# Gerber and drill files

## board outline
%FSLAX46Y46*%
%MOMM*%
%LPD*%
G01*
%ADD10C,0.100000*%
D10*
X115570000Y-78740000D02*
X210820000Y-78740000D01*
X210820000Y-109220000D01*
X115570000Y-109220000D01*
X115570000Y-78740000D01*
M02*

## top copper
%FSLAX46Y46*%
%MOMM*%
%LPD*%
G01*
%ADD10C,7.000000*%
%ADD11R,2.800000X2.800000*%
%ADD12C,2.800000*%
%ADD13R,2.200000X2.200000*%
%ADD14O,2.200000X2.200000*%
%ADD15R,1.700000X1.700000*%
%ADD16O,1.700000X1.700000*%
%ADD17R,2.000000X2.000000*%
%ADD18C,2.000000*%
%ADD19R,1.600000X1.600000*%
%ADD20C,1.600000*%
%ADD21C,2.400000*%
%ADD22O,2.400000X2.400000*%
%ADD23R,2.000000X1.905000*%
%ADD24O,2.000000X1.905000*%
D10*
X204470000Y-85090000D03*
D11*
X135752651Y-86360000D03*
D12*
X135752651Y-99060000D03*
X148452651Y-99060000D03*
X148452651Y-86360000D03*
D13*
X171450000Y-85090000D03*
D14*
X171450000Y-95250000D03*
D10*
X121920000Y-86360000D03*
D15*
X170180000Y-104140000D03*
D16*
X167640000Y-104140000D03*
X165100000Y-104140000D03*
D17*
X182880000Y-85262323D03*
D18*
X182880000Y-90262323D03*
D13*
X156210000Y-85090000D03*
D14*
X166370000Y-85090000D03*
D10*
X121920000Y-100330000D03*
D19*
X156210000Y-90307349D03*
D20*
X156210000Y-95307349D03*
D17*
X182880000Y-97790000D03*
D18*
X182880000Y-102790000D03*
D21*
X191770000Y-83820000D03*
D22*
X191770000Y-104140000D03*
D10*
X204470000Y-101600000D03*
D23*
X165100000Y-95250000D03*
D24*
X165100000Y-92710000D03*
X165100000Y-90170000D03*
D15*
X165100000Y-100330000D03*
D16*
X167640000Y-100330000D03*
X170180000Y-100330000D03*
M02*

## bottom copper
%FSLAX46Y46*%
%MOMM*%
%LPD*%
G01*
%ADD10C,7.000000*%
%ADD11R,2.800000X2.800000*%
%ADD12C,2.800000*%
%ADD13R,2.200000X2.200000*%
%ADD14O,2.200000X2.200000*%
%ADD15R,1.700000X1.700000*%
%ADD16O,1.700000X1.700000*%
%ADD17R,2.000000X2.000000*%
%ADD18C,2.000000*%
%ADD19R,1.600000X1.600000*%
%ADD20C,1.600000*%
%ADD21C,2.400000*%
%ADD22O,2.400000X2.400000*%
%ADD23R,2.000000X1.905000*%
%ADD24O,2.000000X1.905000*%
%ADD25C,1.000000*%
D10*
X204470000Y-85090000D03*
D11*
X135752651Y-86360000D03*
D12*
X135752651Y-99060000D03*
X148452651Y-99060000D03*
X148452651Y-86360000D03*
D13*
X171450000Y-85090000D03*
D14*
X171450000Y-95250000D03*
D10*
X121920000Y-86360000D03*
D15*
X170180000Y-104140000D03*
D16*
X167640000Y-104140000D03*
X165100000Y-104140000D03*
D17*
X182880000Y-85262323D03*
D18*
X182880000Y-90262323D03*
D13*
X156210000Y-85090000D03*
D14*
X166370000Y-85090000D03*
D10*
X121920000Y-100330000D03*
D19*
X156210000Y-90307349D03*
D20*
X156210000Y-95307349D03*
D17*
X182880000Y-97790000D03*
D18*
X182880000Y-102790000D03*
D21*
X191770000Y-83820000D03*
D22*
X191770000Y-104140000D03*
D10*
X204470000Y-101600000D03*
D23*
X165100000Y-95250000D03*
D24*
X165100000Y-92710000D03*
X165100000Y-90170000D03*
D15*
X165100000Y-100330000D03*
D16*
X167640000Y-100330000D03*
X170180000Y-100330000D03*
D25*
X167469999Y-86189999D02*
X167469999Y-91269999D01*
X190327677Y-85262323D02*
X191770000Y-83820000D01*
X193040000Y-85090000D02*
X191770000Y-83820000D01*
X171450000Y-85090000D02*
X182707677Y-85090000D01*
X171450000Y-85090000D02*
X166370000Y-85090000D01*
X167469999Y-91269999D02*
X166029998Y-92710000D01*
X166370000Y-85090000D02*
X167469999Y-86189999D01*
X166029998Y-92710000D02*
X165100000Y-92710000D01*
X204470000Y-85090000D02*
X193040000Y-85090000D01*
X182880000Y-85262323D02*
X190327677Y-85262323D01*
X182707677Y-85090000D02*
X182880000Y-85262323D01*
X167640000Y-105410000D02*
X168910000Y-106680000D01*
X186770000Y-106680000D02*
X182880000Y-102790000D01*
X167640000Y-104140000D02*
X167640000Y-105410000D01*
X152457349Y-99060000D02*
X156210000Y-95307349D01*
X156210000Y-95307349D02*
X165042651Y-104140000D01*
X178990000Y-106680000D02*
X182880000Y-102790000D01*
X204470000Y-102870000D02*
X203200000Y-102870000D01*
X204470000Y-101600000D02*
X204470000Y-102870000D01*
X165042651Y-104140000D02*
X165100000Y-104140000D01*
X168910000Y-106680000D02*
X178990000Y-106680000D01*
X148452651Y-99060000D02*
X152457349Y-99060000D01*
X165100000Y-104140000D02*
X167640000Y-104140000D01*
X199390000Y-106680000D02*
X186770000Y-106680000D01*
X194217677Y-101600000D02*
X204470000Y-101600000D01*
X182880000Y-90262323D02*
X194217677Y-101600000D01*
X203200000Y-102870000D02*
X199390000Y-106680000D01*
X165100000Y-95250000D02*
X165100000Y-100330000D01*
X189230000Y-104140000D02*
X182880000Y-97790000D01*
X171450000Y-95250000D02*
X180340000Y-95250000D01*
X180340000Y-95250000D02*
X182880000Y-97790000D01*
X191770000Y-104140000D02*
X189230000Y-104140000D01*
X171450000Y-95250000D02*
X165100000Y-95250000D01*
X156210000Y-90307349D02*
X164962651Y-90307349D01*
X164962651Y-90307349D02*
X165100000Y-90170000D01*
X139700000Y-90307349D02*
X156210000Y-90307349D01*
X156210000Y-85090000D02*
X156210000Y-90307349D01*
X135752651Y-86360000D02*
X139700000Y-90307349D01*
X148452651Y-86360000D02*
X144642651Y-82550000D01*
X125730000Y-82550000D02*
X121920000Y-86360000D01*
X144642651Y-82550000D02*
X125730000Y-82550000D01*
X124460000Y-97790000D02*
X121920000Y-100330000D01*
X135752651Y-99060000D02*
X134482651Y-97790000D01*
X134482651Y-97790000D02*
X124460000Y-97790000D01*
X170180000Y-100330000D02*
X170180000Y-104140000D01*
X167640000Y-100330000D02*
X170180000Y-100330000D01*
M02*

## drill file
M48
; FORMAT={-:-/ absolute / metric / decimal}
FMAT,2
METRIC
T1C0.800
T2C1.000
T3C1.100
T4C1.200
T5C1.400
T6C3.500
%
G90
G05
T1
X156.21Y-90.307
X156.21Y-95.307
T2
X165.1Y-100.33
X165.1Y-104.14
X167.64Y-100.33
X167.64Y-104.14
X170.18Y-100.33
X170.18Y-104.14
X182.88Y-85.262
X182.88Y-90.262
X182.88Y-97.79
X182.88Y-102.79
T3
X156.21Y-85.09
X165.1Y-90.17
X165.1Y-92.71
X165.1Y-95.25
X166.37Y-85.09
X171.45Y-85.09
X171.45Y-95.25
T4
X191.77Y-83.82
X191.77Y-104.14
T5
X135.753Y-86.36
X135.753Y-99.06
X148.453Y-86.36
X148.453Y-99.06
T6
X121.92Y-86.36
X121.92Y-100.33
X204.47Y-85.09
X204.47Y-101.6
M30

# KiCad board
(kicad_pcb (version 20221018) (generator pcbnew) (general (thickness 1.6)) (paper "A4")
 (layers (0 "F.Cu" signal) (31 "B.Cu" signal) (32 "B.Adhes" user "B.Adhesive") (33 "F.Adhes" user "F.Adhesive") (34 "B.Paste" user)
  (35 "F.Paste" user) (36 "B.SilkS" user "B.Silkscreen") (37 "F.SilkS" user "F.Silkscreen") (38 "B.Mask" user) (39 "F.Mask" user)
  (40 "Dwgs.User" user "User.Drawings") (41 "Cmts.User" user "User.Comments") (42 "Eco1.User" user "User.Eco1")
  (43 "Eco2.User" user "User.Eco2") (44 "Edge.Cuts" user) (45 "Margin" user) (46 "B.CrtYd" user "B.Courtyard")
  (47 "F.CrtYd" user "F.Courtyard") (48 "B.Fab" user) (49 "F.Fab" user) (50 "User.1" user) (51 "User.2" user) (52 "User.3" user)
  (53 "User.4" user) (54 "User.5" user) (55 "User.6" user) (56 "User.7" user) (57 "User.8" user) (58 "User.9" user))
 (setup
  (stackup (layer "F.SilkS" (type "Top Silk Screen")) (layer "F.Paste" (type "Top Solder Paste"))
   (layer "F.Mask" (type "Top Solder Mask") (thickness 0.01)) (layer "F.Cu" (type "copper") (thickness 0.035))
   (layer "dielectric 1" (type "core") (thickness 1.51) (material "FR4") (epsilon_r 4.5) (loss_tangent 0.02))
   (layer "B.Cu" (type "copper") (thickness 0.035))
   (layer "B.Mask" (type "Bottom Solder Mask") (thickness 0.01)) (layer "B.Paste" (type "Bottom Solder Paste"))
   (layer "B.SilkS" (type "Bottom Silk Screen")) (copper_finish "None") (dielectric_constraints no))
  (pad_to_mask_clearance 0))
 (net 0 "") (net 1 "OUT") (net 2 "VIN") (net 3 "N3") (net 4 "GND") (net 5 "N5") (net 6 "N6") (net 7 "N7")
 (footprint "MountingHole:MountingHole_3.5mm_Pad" (layer "F.Cu") (at 204.47 85.09)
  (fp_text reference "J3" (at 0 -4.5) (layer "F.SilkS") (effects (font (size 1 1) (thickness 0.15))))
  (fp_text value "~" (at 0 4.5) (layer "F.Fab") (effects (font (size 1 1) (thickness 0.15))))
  (pad "1" thru_hole circle (at 0 0) (size 7 7) (drill 3.5) (layers "*.Cu" "*.Mask") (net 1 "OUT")))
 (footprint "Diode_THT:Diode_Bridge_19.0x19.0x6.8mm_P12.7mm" (layer "F.Cu") (at 135.752651 86.36)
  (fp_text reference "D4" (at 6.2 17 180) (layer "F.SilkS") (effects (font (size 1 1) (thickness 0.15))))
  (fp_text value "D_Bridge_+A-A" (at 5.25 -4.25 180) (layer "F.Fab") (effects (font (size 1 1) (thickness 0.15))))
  (pad "1" thru_hole rect (at 0 0 180) (size 2.8 2.8) (drill 1.4) (layers "*.Cu" "*.Mask") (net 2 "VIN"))
  (pad "2" thru_hole circle (at 0 12.7 180) (size 2.8 2.8) (drill 1.4) (layers "*.Cu" "*.Mask") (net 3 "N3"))
  (pad "3" thru_hole circle (at 12.7 12.7 180) (size 2.8 2.8) (drill 1.4) (layers "*.Cu" "*.Mask") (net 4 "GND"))
  (pad "4" thru_hole circle (at 12.7 0 180) (size 2.8 2.8) (drill 1.4) (layers "*.Cu" "*.Mask") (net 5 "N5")))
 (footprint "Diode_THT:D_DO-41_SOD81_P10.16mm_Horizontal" (layer "F.Cu") (at 171.45 85.09 -90)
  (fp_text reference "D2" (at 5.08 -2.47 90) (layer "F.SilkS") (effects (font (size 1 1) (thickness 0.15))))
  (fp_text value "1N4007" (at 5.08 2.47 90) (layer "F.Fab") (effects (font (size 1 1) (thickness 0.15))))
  (pad "1" thru_hole rect (at 0 0 270) (size 2.2 2.2) (drill 1.1) (layers "*.Cu" "*.Mask") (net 1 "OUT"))
  (pad "2" thru_hole oval (at 10.16 0 270) (size 2.2 2.2) (drill 1.1) (layers "*.Cu" "*.Mask") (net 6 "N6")))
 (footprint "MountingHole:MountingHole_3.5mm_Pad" (layer "F.Cu") (at 121.92 86.36)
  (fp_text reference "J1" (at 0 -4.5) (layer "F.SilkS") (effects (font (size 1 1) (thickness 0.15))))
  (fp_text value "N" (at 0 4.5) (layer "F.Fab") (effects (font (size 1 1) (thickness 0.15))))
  (pad "1" thru_hole circle (at 0 0) (size 7 7) (drill 3.5) (layers "*.Cu" "*.Mask") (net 5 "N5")))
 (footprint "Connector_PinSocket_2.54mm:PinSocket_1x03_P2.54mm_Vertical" (layer "F.Cu") (at 170.18 104.14 -90)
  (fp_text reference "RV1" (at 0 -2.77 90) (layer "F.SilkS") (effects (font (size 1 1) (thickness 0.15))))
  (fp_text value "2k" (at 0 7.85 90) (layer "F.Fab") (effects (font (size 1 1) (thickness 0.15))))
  (pad "1" thru_hole rect (at 0 0 270) (size 1.7 1.7) (drill 1) (layers "*.Cu" "*.Mask") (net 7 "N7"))
  (pad "2" thru_hole oval (at 0 2.54 270) (size 1.7 1.7) (drill 1) (layers "*.Cu" "*.Mask") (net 4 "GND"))
  (pad "3" thru_hole oval (at 0 5.08 270) (size 1.7 1.7) (drill 1) (layers "*.Cu" "*.Mask") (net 4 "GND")))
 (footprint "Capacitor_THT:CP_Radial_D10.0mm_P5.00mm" (layer "F.Cu") (at 182.88 85.262323 -90)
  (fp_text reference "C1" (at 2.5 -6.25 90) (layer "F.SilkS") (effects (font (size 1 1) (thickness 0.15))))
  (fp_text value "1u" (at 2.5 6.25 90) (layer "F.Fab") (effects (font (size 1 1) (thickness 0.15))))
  (pad "1" thru_hole rect (at 0 0 270) (size 2 2) (drill 1) (layers "*.Cu" "*.Mask") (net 1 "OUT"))
  (pad "2" thru_hole circle (at 5 0 270) (size 2 2) (drill 1) (layers "*.Cu" "*.Mask") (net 4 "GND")))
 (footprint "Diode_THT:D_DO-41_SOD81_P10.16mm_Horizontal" (layer "F.Cu") (at 156.21 85.09)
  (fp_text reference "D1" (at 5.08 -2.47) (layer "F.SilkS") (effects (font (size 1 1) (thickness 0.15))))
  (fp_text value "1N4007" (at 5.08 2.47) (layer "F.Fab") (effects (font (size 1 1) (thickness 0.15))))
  (pad "1" thru_hole rect (at 0 0) (size 2.2 2.2) (drill 1.1) (layers "*.Cu" "*.Mask") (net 2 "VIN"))
  (pad "2" thru_hole oval (at 10.16 0) (size 2.2 2.2) (drill 1.1) (layers "*.Cu" "*.Mask") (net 1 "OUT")))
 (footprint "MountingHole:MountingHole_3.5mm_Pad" (layer "F.Cu") (at 121.92 100.33)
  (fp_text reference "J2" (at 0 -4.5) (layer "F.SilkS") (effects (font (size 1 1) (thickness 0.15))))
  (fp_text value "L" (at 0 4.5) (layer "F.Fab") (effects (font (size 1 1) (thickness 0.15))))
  (pad "1" thru_hole circle (at 0 0) (size 7 7) (drill 3.5) (layers "*.Cu" "*.Mask") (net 3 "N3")))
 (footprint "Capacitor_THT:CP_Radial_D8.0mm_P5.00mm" (layer "F.Cu") (at 156.21 90.307349 -90)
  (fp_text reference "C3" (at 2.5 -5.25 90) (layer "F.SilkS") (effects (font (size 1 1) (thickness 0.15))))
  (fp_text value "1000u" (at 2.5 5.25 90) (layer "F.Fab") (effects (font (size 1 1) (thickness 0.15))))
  (pad "1" thru_hole rect (at 0 0 270) (size 1.6 1.6) (drill 0.8) (layers "*.Cu" "*.Mask") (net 2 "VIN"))
  (pad "2" thru_hole circle (at 5 0 270) (size 1.6 1.6) (drill 0.8) (layers "*.Cu" "*.Mask") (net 4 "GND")))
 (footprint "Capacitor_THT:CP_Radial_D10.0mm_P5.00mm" (layer "F.Cu") (at 182.88 97.79 -90)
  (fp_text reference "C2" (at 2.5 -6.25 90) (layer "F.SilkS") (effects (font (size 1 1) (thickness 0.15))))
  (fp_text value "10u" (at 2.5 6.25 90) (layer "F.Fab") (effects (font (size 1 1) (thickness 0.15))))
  (pad "1" thru_hole rect (at 0 0 270) (size 2 2) (drill 1) (layers "*.Cu" "*.Mask") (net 6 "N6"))
  (pad "2" thru_hole circle (at 5 0 270) (size 2 2) (drill 1) (layers "*.Cu" "*.Mask") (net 4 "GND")))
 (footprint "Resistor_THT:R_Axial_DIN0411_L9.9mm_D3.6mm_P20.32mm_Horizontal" (layer "F.Cu") (at 191.77 83.82 -90)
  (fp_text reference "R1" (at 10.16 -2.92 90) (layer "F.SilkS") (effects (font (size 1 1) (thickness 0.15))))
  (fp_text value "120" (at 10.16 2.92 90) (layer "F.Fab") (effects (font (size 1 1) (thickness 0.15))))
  (pad "1" thru_hole circle (at 0 0 270) (size 2.4 2.4) (drill 1.2) (layers "*.Cu" "*.Mask") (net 1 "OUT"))
  (pad "2" thru_hole oval (at 20.32 0 270) (size 2.4 2.4) (drill 1.2) (layers "*.Cu" "*.Mask") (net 6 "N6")))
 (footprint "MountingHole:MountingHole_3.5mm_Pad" (layer "F.Cu") (at 204.47 101.6)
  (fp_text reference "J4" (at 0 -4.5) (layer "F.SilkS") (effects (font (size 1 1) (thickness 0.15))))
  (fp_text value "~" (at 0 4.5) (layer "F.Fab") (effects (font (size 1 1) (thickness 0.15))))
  (pad "1" thru_hole circle (at 0 0) (size 7 7) (drill 3.5) (layers "*.Cu" "*.Mask") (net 4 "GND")))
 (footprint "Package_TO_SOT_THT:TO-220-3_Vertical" (layer "F.Cu") (at 165.1 95.25 90)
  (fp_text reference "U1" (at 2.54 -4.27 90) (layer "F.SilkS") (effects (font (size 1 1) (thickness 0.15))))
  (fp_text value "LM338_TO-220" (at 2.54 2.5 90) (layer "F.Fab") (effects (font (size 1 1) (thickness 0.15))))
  (pad "1" thru_hole rect (at 0 0 90) (size 1.905 2) (drill 1.1) (layers "*.Cu" "*.Mask") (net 6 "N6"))
  (pad "2" thru_hole oval (at 2.54 0 90) (size 1.905 2) (drill 1.1) (layers "*.Cu" "*.Mask") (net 1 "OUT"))
  (pad "3" thru_hole oval (at 5.08 0 90) (size 1.905 2) (drill 1.1) (layers "*.Cu" "*.Mask") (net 2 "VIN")))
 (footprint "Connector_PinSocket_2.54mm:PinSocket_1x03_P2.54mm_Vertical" (layer "F.Cu") (at 165.1 100.33 90)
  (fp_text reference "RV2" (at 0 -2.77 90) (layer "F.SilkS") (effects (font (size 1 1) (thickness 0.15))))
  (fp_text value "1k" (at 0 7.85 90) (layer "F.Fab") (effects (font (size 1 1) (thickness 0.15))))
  (pad "1" thru_hole rect (at 0 0 90) (size 1.7 1.7) (drill 1) (layers "*.Cu" "*.Mask") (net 6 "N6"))
  (pad "2" thru_hole oval (at 0 2.54 90) (size 1.7 1.7) (drill 1) (layers "*.Cu" "*.Mask") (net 7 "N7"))
  (pad "3" thru_hole oval (at 0 5.08 90) (size 1.7 1.7) (drill 1) (layers "*.Cu" "*.Mask") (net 7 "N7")))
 (gr_rect (start 115.57 78.74) (end 210.82 109.22) (stroke (width 0.1) (type default)) (fill none) (layer "Edge.Cuts"))
 (segment (start 167.469999 86.189999) (end 167.469999 91.269999) (width 1) (layer "B.Cu") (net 1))
 (segment (start 190.327677 85.262323) (end 191.77 83.82) (width 1) (layer "B.Cu") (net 1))
 (segment (start 193.04 85.09) (end 191.77 83.82) (width 1) (layer "B.Cu") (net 1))
 (segment (start 171.45 85.09) (end 182.707677 85.09) (width 1) (layer "B.Cu") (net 1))
 (segment (start 171.45 85.09) (end 166.37 85.09) (width 1) (layer "B.Cu") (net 1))
 (segment (start 167.469999 91.269999) (end 166.029998 92.71) (width 1) (layer "B.Cu") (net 1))
 (segment (start 166.37 85.09) (end 167.469999 86.189999) (width 1) (layer "B.Cu") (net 1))
 (segment (start 166.029998 92.71) (end 165.1 92.71) (width 1) (layer "B.Cu") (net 1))
 (segment (start 204.47 85.09) (end 193.04 85.09) (width 1) (layer "B.Cu") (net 1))
 (segment (start 182.88 85.262323) (end 190.327677 85.262323) (width 1) (layer "B.Cu") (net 1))
 (segment (start 182.707677 85.09) (end 182.88 85.262323) (width 1) (layer "B.Cu") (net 1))
 (segment (start 167.64 105.41) (end 168.91 106.68) (width 1) (layer "B.Cu") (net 4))
 (segment (start 186.77 106.68) (end 182.88 102.79) (width 1) (layer "B.Cu") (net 4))
 (segment (start 167.64 104.14) (end 167.64 105.41) (width 1) (layer "B.Cu") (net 4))
 (segment (start 152.457349 99.06) (end 156.21 95.307349) (width 1) (layer "B.Cu") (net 4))
 (segment (start 156.21 95.307349) (end 165.042651 104.14) (width 1) (layer "B.Cu") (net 4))
 (segment (start 178.99 106.68) (end 182.88 102.79) (width 1) (layer "B.Cu") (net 4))
 (segment (start 204.47 102.87) (end 203.2 102.87) (width 1) (layer "B.Cu") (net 4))
 (segment (start 204.47 101.6) (end 204.47 102.87) (width 1) (layer "B.Cu") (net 4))
 (segment (start 165.042651 104.14) (end 165.1 104.14) (width 1) (layer "B.Cu") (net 4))
 (segment (start 168.91 106.68) (end 178.99 106.68) (width 1) (layer "B.Cu") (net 4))
 (segment (start 148.452651 99.06) (end 152.457349 99.06) (width 1) (layer "B.Cu") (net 4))
 (segment (start 165.1 104.14) (end 167.64 104.14) (width 1) (layer "B.Cu") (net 4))
 (segment (start 199.39 106.68) (end 186.77 106.68) (width 1) (layer "B.Cu") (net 4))
 (segment (start 194.217677 101.6) (end 204.47 101.6) (width 1) (layer "B.Cu") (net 4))
 (segment (start 182.88 90.262323) (end 194.217677 101.6) (width 1) (layer "B.Cu") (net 4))
 (segment (start 203.2 102.87) (end 199.39 106.68) (width 1) (layer "B.Cu") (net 4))
 (segment (start 165.1 95.25) (end 165.1 100.33) (width 1) (layer "B.Cu") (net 6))
 (segment (start 189.23 104.14) (end 182.88 97.79) (width 1) (layer "B.Cu") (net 6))
 (segment (start 171.45 95.25) (end 180.34 95.25) (width 1) (layer "B.Cu") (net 6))
 (segment (start 180.34 95.25) (end 182.88 97.79) (width 1) (layer "B.Cu") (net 6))
 (segment (start 191.77 104.14) (end 189.23 104.14) (width 1) (layer "B.Cu") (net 6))
 (segment (start 171.45 95.25) (end 165.1 95.25) (width 1) (layer "B.Cu") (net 6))
 (segment (start 156.21 90.307349) (end 164.962651 90.307349) (width 1) (layer "B.Cu") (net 2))
 (segment (start 164.962651 90.307349) (end 165.1 90.17) (width 1) (layer "B.Cu") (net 2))
 (segment (start 139.7 90.307349) (end 156.21 90.307349) (width 1) (layer "B.Cu") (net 2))
 (segment (start 156.21 85.09) (end 156.21 90.307349) (width 1) (layer "B.Cu") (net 2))
 (segment (start 135.752651 86.36) (end 139.7 90.307349) (width 1) (layer "B.Cu") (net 2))
 (segment (start 148.452651 86.36) (end 144.642651 82.55) (width 1) (layer "B.Cu") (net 5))
 (segment (start 125.73 82.55) (end 121.92 86.36) (width 1) (layer "B.Cu") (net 5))
 (segment (start 144.642651 82.55) (end 125.73 82.55) (width 1) (layer "B.Cu") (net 5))
 (segment (start 124.46 97.79) (end 121.92 100.33) (width 1) (layer "B.Cu") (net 3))
 (segment (start 135.752651 99.06) (end 134.482651 97.79) (width 1) (layer "B.Cu") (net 3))
 (segment (start 134.482651 97.79) (end 124.46 97.79) (width 1) (layer "B.Cu") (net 3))
 (segment (start 170.18 100.33) (end 170.18 104.14) (width 1) (layer "B.Cu") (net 7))
 (segment (start 167.64 100.33) (end 170.18 100.33) (width 1) (layer "B.Cu") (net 7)))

